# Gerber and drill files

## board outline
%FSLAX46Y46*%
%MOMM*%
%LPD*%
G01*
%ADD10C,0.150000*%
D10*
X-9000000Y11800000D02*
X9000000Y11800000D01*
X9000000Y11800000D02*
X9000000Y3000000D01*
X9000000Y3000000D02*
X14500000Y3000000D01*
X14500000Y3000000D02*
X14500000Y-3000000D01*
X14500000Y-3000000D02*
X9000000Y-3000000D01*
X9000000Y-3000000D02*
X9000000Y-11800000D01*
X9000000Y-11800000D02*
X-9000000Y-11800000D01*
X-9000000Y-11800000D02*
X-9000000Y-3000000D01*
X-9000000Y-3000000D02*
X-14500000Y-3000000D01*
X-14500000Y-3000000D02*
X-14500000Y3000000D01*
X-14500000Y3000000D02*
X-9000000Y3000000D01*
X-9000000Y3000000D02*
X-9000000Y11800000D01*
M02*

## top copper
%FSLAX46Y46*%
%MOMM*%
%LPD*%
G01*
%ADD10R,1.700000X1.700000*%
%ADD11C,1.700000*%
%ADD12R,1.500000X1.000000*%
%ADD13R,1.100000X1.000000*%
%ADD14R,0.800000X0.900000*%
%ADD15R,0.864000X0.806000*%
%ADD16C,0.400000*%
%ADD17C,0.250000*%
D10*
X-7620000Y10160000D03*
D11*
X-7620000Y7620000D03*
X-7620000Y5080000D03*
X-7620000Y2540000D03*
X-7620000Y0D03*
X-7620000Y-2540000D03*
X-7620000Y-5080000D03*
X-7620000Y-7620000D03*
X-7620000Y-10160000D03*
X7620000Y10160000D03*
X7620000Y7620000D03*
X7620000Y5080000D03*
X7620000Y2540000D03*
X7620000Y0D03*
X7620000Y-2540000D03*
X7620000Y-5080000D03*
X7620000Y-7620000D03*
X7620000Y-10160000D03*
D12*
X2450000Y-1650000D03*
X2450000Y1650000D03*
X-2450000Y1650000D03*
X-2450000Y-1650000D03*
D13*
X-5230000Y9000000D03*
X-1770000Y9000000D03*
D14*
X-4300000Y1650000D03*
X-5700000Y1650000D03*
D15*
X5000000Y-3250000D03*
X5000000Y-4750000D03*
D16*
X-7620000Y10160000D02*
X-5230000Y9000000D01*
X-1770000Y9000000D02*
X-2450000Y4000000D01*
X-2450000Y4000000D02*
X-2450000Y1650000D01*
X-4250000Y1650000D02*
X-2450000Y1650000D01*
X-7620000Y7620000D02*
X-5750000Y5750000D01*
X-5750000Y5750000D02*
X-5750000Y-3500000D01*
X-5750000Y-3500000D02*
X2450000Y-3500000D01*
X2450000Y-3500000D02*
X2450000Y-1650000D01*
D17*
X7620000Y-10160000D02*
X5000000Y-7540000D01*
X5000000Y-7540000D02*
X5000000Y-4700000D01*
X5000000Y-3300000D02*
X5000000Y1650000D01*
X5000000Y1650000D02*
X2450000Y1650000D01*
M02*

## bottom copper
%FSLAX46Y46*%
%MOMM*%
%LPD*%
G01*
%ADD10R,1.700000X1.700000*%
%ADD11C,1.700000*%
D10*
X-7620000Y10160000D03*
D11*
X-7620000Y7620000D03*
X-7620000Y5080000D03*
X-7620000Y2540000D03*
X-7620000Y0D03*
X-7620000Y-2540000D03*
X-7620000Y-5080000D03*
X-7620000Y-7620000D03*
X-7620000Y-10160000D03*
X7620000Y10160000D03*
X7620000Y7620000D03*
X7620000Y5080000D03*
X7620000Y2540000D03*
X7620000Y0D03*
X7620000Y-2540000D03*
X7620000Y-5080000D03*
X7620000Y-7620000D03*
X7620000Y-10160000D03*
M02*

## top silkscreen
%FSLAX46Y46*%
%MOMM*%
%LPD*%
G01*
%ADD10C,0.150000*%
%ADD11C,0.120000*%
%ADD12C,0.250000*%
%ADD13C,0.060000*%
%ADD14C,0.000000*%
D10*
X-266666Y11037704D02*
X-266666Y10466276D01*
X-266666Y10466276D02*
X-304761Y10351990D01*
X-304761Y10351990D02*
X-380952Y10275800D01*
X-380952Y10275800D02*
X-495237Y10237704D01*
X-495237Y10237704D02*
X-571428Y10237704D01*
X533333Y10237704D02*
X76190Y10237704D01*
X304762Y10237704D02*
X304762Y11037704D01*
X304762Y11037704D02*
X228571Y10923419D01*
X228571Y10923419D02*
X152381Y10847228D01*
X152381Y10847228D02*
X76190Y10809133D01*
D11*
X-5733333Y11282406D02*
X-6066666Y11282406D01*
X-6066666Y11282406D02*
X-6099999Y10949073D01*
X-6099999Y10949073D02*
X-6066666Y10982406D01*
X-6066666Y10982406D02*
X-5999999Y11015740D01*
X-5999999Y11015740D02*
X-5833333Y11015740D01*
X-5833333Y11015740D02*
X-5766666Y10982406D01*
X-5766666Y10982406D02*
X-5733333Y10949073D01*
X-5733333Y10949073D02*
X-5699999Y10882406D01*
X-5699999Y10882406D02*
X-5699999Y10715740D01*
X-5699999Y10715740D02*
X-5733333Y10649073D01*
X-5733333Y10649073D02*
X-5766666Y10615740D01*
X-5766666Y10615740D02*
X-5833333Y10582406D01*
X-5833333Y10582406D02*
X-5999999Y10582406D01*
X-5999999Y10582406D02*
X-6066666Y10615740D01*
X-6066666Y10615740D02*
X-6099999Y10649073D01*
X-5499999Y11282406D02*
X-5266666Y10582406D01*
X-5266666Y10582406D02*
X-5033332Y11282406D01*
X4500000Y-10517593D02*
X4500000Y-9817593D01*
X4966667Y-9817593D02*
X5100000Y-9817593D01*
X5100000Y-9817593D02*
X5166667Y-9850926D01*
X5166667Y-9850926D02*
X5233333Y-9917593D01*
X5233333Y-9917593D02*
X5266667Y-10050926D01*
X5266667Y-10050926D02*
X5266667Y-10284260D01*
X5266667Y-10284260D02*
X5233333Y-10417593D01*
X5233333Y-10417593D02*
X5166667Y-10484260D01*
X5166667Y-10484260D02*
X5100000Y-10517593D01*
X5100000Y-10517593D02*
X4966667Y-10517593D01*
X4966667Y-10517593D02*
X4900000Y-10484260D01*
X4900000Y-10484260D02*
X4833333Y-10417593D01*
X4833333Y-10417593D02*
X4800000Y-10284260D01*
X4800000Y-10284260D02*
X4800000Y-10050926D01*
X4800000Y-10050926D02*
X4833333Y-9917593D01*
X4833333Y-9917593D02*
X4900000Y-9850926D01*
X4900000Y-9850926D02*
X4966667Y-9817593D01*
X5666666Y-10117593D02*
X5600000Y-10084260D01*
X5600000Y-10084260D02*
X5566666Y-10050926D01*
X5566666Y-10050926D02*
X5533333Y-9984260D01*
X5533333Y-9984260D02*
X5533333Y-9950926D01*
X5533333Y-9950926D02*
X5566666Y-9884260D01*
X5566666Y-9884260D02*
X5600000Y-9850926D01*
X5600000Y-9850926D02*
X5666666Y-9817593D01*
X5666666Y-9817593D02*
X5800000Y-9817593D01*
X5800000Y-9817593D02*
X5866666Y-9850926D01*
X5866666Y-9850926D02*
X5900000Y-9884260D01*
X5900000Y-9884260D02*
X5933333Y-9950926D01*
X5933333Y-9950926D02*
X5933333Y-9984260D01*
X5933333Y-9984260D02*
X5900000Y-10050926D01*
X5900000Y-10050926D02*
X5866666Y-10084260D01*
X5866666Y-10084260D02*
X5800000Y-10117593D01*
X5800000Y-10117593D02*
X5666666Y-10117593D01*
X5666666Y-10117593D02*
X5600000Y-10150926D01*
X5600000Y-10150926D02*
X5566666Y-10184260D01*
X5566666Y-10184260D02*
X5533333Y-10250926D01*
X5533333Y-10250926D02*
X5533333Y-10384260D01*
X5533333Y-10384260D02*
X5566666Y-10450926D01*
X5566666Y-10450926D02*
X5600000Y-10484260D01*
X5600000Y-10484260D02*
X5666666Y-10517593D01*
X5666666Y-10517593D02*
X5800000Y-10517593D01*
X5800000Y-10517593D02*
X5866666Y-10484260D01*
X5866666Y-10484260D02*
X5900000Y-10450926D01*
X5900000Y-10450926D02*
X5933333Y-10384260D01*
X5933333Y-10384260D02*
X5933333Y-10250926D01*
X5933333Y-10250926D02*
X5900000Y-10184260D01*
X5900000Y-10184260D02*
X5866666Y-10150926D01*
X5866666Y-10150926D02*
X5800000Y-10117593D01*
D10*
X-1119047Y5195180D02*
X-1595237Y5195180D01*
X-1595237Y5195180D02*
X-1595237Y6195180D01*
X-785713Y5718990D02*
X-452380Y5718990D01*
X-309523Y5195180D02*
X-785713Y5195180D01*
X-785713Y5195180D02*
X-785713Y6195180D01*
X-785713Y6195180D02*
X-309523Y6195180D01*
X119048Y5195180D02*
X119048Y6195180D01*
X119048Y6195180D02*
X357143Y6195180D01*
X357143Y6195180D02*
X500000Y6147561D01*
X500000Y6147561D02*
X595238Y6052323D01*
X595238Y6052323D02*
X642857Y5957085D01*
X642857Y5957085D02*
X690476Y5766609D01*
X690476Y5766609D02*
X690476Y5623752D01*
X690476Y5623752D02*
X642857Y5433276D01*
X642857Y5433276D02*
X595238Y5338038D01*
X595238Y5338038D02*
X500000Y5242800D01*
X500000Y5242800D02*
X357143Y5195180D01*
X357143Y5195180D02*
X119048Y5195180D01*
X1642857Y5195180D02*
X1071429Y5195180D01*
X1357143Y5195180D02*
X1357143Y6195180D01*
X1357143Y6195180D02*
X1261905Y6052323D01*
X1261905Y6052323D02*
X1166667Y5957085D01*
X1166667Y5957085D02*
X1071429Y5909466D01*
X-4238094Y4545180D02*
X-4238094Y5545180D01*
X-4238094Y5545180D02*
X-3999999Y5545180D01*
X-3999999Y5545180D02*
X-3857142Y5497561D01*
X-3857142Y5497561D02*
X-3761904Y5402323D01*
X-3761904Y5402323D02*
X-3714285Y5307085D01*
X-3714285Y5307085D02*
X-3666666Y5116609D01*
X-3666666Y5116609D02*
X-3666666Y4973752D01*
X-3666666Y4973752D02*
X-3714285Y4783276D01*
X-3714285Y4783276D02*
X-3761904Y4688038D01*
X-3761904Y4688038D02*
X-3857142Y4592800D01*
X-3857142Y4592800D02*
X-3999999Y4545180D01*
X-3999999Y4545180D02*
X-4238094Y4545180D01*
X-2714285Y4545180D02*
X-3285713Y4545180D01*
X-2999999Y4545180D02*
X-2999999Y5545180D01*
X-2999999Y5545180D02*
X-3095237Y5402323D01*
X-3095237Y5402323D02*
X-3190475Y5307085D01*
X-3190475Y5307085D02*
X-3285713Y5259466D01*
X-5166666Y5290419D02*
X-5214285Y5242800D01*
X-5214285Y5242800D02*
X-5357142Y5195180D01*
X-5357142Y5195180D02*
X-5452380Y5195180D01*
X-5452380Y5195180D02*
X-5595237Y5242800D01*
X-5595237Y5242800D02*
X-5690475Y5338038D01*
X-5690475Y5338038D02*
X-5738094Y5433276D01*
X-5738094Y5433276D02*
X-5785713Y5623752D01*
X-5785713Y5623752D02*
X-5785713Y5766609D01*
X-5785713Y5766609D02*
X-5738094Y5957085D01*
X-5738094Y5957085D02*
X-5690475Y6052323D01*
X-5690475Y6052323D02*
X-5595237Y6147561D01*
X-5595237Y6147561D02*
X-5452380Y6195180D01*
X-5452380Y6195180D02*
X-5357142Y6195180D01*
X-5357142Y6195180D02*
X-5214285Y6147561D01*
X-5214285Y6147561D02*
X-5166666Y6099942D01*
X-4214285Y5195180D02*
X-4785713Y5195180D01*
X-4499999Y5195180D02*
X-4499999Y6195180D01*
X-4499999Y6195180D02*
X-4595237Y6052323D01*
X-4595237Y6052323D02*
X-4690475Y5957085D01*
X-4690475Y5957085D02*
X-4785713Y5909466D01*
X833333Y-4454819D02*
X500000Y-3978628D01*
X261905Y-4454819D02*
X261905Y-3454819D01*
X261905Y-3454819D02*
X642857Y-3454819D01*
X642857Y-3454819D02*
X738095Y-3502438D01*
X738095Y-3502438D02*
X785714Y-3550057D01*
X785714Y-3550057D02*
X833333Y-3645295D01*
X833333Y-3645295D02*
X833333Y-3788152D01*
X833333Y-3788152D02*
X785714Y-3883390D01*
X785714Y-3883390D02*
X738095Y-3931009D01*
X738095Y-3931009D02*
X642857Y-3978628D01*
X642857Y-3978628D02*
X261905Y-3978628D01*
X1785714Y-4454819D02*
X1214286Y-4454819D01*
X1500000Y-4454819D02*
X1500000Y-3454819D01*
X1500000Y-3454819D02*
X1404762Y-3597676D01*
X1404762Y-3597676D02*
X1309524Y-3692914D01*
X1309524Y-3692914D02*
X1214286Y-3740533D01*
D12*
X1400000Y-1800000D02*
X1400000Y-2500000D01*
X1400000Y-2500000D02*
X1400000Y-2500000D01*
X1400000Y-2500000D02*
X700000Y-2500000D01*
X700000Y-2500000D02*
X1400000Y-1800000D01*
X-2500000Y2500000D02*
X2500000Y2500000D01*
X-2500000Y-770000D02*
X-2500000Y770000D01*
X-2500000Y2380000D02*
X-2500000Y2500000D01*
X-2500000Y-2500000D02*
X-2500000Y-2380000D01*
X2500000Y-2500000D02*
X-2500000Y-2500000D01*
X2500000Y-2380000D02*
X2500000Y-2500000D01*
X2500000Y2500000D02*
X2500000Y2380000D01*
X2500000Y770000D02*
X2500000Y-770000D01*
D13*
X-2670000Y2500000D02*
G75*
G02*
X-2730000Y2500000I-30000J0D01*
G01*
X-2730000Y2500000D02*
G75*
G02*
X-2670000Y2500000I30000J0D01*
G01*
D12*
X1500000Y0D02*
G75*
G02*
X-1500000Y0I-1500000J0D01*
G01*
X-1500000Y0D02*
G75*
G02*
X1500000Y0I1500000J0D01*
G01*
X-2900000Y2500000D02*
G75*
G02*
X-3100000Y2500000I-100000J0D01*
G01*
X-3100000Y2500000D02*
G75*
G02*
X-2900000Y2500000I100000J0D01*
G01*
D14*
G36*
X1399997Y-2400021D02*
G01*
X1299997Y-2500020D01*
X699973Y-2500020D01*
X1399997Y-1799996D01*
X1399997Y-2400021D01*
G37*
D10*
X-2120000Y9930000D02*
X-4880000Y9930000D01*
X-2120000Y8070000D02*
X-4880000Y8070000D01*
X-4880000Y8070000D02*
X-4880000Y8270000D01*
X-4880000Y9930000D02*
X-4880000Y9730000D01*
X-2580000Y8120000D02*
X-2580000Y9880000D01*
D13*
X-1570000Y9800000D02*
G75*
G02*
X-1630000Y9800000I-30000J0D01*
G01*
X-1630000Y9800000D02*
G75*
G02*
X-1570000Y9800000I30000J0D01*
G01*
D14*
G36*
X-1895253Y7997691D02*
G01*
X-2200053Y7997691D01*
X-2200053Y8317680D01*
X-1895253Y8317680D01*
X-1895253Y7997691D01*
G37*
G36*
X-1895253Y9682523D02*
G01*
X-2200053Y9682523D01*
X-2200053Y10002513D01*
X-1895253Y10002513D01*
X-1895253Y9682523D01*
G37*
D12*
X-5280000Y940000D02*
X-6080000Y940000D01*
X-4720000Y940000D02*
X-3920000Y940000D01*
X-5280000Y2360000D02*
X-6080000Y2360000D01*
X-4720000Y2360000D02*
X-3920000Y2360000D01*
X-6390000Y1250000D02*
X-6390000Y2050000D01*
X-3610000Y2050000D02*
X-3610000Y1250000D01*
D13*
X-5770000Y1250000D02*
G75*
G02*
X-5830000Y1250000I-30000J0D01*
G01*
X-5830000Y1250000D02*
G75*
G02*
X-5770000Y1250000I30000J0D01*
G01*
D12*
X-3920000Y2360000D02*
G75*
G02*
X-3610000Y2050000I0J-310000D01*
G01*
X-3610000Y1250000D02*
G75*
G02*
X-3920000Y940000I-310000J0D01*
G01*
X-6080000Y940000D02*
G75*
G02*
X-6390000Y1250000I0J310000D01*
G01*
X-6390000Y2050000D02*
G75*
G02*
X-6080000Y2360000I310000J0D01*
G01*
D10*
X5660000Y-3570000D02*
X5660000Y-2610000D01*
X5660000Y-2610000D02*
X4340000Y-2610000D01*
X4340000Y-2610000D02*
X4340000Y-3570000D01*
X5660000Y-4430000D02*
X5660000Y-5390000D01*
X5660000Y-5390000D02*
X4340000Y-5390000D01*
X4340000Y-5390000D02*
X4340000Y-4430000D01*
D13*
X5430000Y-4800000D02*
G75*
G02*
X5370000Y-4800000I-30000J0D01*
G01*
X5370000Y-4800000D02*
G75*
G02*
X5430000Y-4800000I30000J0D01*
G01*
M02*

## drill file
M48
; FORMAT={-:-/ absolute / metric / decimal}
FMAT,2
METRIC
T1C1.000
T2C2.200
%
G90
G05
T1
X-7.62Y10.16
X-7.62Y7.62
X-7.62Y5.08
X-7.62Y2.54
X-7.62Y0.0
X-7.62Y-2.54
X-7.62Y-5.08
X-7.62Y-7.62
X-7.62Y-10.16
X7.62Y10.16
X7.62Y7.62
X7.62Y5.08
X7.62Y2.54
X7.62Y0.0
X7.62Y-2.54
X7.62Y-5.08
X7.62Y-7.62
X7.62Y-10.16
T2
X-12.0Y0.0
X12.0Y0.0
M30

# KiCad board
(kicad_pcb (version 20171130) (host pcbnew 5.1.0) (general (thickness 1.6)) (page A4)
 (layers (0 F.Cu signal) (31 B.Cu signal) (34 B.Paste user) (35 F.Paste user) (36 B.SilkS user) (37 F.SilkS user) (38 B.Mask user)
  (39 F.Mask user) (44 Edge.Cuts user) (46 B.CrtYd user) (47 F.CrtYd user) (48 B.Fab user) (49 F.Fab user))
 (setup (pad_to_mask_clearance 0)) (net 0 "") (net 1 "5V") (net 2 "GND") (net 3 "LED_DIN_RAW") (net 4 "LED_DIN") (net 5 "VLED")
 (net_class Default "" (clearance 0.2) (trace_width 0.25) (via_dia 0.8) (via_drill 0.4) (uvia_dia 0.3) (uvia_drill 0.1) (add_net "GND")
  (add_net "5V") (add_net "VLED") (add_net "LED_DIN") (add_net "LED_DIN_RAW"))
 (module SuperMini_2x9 (layer F.Cu) (at 0 0)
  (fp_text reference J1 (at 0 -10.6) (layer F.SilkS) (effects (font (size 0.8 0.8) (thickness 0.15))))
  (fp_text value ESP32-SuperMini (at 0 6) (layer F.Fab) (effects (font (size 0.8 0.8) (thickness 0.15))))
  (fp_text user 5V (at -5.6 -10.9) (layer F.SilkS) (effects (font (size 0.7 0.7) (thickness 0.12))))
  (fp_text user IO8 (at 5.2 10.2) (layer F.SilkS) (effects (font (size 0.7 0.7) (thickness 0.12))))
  (pad "5V" thru_hole rect (at -7.62 -10.16) (size 1.7 1.7) (drill 1.0) (layers *.Cu *.Mask) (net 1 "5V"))
  (pad "GND" thru_hole circle (at -7.62 -7.62) (size 1.7 1.7) (drill 1.0) (layers *.Cu *.Mask) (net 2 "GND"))
  (pad "3V3" thru_hole circle (at -7.62 -5.08) (size 1.7 1.7) (drill 1.0) (layers *.Cu *.Mask))
  (pad "IO14" thru_hole circle (at -7.62 -2.54) (size 1.7 1.7) (drill 1.0) (layers *.Cu *.Mask))
  (pad "IO13" thru_hole circle (at -7.62 0.0) (size 1.7 1.7) (drill 1.0) (layers *.Cu *.Mask))
  (pad "IO12" thru_hole circle (at -7.62 2.54) (size 1.7 1.7) (drill 1.0) (layers *.Cu *.Mask))
  (pad "IO11" thru_hole circle (at -7.62 5.08) (size 1.7 1.7) (drill 1.0) (layers *.Cu *.Mask))
  (pad "IO10" thru_hole circle (at -7.62 7.62) (size 1.7 1.7) (drill 1.0) (layers *.Cu *.Mask))
  (pad "IO9" thru_hole circle (at -7.62 10.16) (size 1.7 1.7) (drill 1.0) (layers *.Cu *.Mask))
  (pad "IO24" thru_hole circle (at 7.62 -10.16) (size 1.7 1.7) (drill 1.0) (layers *.Cu *.Mask))
  (pad "IO23" thru_hole circle (at 7.62 -7.62) (size 1.7 1.7) (drill 1.0) (layers *.Cu *.Mask))
  (pad "IO0" thru_hole circle (at 7.62 -5.08) (size 1.7 1.7) (drill 1.0) (layers *.Cu *.Mask))
  (pad "IO1" thru_hole circle (at 7.62 -2.54) (size 1.7 1.7) (drill 1.0) (layers *.Cu *.Mask))
  (pad "IO2" thru_hole circle (at 7.62 0.0) (size 1.7 1.7) (drill 1.0) (layers *.Cu *.Mask))
  (pad "IO3" thru_hole circle (at 7.62 2.54) (size 1.7 1.7) (drill 1.0) (layers *.Cu *.Mask))
  (pad "IO4" thru_hole circle (at 7.62 5.08) (size 1.7 1.7) (drill 1.0) (layers *.Cu *.Mask))
  (pad "IO5" thru_hole circle (at 7.62 7.62) (size 1.7 1.7) (drill 1.0) (layers *.Cu *.Mask))
  (pad "IO8" thru_hole circle (at 7.62 10.16) (size 1.7 1.7) (drill 1.0) (layers *.Cu *.Mask) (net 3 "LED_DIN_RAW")))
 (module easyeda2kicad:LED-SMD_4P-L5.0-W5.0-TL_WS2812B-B (layer F.Cu) (at 0 0 0)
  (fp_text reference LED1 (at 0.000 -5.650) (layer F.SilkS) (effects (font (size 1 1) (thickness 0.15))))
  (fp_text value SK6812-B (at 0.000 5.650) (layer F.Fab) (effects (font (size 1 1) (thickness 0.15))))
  (fp_line (start 1.40 1.80) (end 1.40 2.50) (layer F.SilkS) (width 0.25))
  (fp_line (start 1.40 2.50) (end 1.40 2.50) (layer F.SilkS) (width 0.25))
  (fp_line (start 1.40 2.50) (end 0.70 2.50) (layer F.SilkS) (width 0.25))
  (fp_line (start 0.70 2.50) (end 1.40 1.80) (layer F.SilkS) (width 0.25))
  (fp_line (start -2.50 -2.50) (end 2.50 -2.50) (layer F.SilkS) (width 0.25))
  (fp_line (start -2.50 0.77) (end -2.50 -0.77) (layer F.SilkS) (width 0.25))
  (fp_line (start -2.50 -2.38) (end -2.50 -2.50) (layer F.SilkS) (width 0.25))
  (fp_line (start -2.50 2.50) (end -2.50 2.38) (layer F.SilkS) (width 0.25))
  (fp_line (start 2.50 2.50) (end -2.50 2.50) (layer F.SilkS) (width 0.25))
  (fp_line (start 2.50 2.38) (end 2.50 2.50) (layer F.SilkS) (width 0.25))
  (fp_line (start 2.50 -2.50) (end 2.50 -2.38) (layer F.SilkS) (width 0.25))
  (fp_line (start 2.50 -0.77) (end 2.50 0.77) (layer F.SilkS) (width 0.25))
  (pad 3 smd rect (at 2.45 1.65 180.0) (size 1.500 1.000) (layers F.Cu F.Paste F.Mask) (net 2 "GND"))
  (pad 4 smd rect (at 2.45 -1.65 180.0) (size 1.500 1.000) (layers F.Cu F.Paste F.Mask) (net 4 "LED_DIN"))
  (pad 1 smd rect (at -2.45 -1.65 180.0) (size 1.500 1.000) (layers F.Cu F.Paste F.Mask) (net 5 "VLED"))
  (pad 2 smd rect (at -2.45 1.65 180.0) (size 1.500 1.000) (layers F.Cu F.Paste F.Mask))
  (fp_circle (center -2.70 -2.50) (end -2.67 -2.50) (layer F.SilkS) (width 0.06))
  (fp_circle (center 0.00 0.00) (end 1.50 0.00) (layer F.SilkS) (width 0.25))
  (fp_circle (center -3.00 -2.50) (end -2.90 -2.50) (layer F.SilkS) (width 0.25))
  (fp_poly
   (pts (xy 1.399997 1.799996) (xy 1.399997 2.400021) (xy 1.299997 2.500020) (xy 0.699973 2.500020) (xy 1.399997 1.799996))
   (stroke (width 0) (type solid)) (fill solid) (layer "F.SilkS")))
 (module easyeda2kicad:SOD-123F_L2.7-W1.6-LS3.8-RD (layer F.Cu) (at -3.5 -9 180)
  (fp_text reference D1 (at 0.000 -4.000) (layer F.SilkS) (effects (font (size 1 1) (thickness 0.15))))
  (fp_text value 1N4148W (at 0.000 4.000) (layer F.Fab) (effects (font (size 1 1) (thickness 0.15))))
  (fp_line (start -1.38 0.93) (end 1.38 0.93) (layer F.SilkS) (width 0.15))
  (fp_line (start -1.38 -0.93) (end 1.38 -0.93) (layer F.SilkS) (width 0.15))
  (fp_line (start 1.38 -0.93) (end 1.38 -0.73) (layer F.SilkS) (width 0.15))
  (fp_line (start 1.38 0.93) (end 1.38 0.73) (layer F.SilkS) (width 0.15))
  (fp_line (start -0.92 -0.88) (end -0.92 0.88) (layer F.SilkS) (width 0.15))
  (pad 2 smd rect (at 1.73 0.00 180.0) (size 1.100 1.000) (layers F.Cu F.Paste F.Mask) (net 1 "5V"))
  (pad 1 smd rect (at -1.73 0.00 180.0) (size 1.100 1.000) (layers F.Cu F.Paste F.Mask) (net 5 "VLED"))
  (fp_circle (center -1.90 0.80) (end -1.87 0.80) (layer F.SilkS) (width 0.06))
  (fp_poly
   (pts (xy -1.299947 -1.002309) (xy -1.299947 -0.682320) (xy -1.604747 -0.682320) (xy -1.604747 -1.002309) (xy -1.299947 -1.002309))
   (stroke (width 0) (type solid)) (fill solid) (layer "F.SilkS"))
  (fp_poly
   (pts (xy -1.299947 1.002513) (xy -1.299947 0.682523) (xy -1.604747 0.682523) (xy -1.604747 1.002513) (xy -1.299947 1.002513))
   (stroke (width 0) (type solid)) (fill solid) (layer "F.SilkS")))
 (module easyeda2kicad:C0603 (layer F.Cu) (at -5 -1.65 0)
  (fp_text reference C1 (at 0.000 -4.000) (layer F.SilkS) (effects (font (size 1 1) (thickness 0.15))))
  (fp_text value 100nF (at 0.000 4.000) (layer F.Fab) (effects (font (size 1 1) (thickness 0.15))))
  (fp_line (start -0.28 0.71) (end -1.08 0.71) (layer F.SilkS) (width 0.25))
  (fp_line (start 0.28 0.71) (end 1.08 0.71) (layer F.SilkS) (width 0.25))
  (fp_line (start -0.28 -0.71) (end -1.08 -0.71) (layer F.SilkS) (width 0.25))
  (fp_line (start 0.28 -0.71) (end 1.08 -0.71) (layer F.SilkS) (width 0.25))
  (fp_line (start -1.39 0.40) (end -1.39 -0.40) (layer F.SilkS) (width 0.25))
  (fp_line (start 1.39 -0.40) (end 1.39 0.40) (layer F.SilkS) (width 0.25))
  (pad 2 smd rect (at 0.70 0.00 0.0) (size 0.800 0.900) (layers F.Cu F.Paste F.Mask) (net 5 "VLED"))
  (pad 1 smd rect (at -0.70 0.00 0.0) (size 0.800 0.900) (layers F.Cu F.Paste F.Mask) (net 2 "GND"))
  (fp_circle (center -0.80 0.40) (end -0.77 0.40) (layer F.SilkS) (width 0.06))
  (fp_arc (start 1.08 -0.40) (end 1.39 -0.40) (angle -90.00) (layer F.SilkS) (width 0.25))
  (fp_arc (start 1.08 0.40) (end 1.08 0.71) (angle -90.00) (layer F.SilkS) (width 0.25))
  (fp_arc (start -1.08 0.40) (end -1.39 0.40) (angle -90.00) (layer F.SilkS) (width 0.25))
  (fp_arc (start -1.08 -0.40) (end -1.08 -0.71) (angle -90.00) (layer F.SilkS) (width 0.25)))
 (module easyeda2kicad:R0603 (layer F.Cu) (at 5 4 90)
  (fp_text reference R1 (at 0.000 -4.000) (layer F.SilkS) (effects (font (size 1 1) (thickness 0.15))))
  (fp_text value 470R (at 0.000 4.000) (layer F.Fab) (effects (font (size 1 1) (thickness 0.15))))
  (fp_line (start 0.43 0.66) (end 1.39 0.66) (layer F.SilkS) (width 0.15))
  (fp_line (start 1.39 0.66) (end 1.39 -0.66) (layer F.SilkS) (width 0.15))
  (fp_line (start 1.39 -0.66) (end 0.43 -0.66) (layer F.SilkS) (width 0.15))
  (fp_line (start -0.43 0.66) (end -1.39 0.66) (layer F.SilkS) (width 0.15))
  (fp_line (start -1.39 0.66) (end -1.39 -0.66) (layer F.SilkS) (width 0.15))
  (fp_line (start -1.39 -0.66) (end -0.43 -0.66) (layer F.SilkS) (width 0.15))
  (pad 2 smd rect (at 0.75 0.00 90.0) (size 0.806 0.864) (layers F.Cu F.Paste F.Mask) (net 4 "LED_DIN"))
  (pad 1 smd rect (at -0.75 0.00 90.0) (size 0.806 0.864) (layers F.Cu F.Paste F.Mask) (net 3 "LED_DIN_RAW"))
  (fp_circle (center -0.80 0.40) (end -0.77 0.40) (layer F.SilkS) (width 0.06)))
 (segment (start -7.62 -10.16) (end -5.23 -9) (width 0.4) (layer F.Cu) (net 1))
 (segment (start -1.77 -9) (end -2.45 -4) (width 0.4) (layer F.Cu) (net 5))
 (segment (start -2.45 -4) (end -2.45 -1.65) (width 0.4) (layer F.Cu) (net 5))
 (segment (start -4.25 -1.65) (end -2.45 -1.65) (width 0.4) (layer F.Cu) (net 5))
 (segment (start -7.62 -7.62) (end -5.75 -5.75) (width 0.4) (layer F.Cu) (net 2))
 (segment (start -5.75 -5.75) (end -5.75 3.5) (width 0.4) (layer F.Cu) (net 2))
 (segment (start -5.75 3.5) (end 2.45 3.5) (width 0.4) (layer F.Cu) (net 2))
 (segment (start 2.45 3.5) (end 2.45 1.65) (width 0.4) (layer F.Cu) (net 2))
 (segment (start 7.62 10.16) (end 5 7.54) (width 0.25) (layer F.Cu) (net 3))
 (segment (start 5 7.54) (end 5 4.7) (width 0.25) (layer F.Cu) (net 3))
 (segment (start 5 3.3) (end 5 -1.65) (width 0.25) (layer F.Cu) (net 4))
 (segment (start 5 -1.65) (end 2.45 -1.65) (width 0.25) (layer F.Cu) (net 4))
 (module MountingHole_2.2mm (layer F.Cu) (at -12 0)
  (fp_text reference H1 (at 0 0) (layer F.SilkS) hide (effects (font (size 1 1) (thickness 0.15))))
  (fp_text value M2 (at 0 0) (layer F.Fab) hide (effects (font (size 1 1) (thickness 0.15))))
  (pad "" np_thru_hole circle (at 0 0) (size 2.2 2.2) (drill 2.2) (layers *.Cu *.Mask)))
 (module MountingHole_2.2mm (layer F.Cu) (at 12 0)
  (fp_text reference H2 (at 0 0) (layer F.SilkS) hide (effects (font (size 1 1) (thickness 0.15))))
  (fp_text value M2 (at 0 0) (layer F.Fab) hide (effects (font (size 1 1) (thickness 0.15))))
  (pad "" np_thru_hole circle (at 0 0) (size 2.2 2.2) (drill 2.2) (layers *.Cu *.Mask)))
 (gr_line (start -9.0 -11.8) (end 9.0 -11.8) (layer Edge.Cuts) (width 0.15))
 (gr_line (start 9.0 -11.8) (end 9.0 -3.0) (layer Edge.Cuts) (width 0.15))
 (gr_line (start 9.0 -3.0) (end 14.5 -3.0) (layer Edge.Cuts) (width 0.15))
 (gr_line (start 14.5 -3.0) (end 14.5 3.0) (layer Edge.Cuts) (width 0.15))
 (gr_line (start 14.5 3.0) (end 9.0 3.0) (layer Edge.Cuts) (width 0.15))
 (gr_line (start 9.0 3.0) (end 9.0 11.8) (layer Edge.Cuts) (width 0.15))
 (gr_line (start 9.0 11.8) (end -9.0 11.8) (layer Edge.Cuts) (width 0.15))
 (gr_line (start -9.0 11.8) (end -9.0 3.0) (layer Edge.Cuts) (width 0.15))
 (gr_line (start -9.0 3.0) (end -14.5 3.0) (layer Edge.Cuts) (width 0.15))
 (gr_line (start -14.5 3.0) (end -14.5 -3.0) (layer Edge.Cuts) (width 0.15))
 (gr_line (start -14.5 -3.0) (end -9.0 -3.0) (layer Edge.Cuts) (width 0.15))
 (gr_line (start -9.0 -3.0) (end -9.0 -11.8) (layer Edge.Cuts) (width 0.15)))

